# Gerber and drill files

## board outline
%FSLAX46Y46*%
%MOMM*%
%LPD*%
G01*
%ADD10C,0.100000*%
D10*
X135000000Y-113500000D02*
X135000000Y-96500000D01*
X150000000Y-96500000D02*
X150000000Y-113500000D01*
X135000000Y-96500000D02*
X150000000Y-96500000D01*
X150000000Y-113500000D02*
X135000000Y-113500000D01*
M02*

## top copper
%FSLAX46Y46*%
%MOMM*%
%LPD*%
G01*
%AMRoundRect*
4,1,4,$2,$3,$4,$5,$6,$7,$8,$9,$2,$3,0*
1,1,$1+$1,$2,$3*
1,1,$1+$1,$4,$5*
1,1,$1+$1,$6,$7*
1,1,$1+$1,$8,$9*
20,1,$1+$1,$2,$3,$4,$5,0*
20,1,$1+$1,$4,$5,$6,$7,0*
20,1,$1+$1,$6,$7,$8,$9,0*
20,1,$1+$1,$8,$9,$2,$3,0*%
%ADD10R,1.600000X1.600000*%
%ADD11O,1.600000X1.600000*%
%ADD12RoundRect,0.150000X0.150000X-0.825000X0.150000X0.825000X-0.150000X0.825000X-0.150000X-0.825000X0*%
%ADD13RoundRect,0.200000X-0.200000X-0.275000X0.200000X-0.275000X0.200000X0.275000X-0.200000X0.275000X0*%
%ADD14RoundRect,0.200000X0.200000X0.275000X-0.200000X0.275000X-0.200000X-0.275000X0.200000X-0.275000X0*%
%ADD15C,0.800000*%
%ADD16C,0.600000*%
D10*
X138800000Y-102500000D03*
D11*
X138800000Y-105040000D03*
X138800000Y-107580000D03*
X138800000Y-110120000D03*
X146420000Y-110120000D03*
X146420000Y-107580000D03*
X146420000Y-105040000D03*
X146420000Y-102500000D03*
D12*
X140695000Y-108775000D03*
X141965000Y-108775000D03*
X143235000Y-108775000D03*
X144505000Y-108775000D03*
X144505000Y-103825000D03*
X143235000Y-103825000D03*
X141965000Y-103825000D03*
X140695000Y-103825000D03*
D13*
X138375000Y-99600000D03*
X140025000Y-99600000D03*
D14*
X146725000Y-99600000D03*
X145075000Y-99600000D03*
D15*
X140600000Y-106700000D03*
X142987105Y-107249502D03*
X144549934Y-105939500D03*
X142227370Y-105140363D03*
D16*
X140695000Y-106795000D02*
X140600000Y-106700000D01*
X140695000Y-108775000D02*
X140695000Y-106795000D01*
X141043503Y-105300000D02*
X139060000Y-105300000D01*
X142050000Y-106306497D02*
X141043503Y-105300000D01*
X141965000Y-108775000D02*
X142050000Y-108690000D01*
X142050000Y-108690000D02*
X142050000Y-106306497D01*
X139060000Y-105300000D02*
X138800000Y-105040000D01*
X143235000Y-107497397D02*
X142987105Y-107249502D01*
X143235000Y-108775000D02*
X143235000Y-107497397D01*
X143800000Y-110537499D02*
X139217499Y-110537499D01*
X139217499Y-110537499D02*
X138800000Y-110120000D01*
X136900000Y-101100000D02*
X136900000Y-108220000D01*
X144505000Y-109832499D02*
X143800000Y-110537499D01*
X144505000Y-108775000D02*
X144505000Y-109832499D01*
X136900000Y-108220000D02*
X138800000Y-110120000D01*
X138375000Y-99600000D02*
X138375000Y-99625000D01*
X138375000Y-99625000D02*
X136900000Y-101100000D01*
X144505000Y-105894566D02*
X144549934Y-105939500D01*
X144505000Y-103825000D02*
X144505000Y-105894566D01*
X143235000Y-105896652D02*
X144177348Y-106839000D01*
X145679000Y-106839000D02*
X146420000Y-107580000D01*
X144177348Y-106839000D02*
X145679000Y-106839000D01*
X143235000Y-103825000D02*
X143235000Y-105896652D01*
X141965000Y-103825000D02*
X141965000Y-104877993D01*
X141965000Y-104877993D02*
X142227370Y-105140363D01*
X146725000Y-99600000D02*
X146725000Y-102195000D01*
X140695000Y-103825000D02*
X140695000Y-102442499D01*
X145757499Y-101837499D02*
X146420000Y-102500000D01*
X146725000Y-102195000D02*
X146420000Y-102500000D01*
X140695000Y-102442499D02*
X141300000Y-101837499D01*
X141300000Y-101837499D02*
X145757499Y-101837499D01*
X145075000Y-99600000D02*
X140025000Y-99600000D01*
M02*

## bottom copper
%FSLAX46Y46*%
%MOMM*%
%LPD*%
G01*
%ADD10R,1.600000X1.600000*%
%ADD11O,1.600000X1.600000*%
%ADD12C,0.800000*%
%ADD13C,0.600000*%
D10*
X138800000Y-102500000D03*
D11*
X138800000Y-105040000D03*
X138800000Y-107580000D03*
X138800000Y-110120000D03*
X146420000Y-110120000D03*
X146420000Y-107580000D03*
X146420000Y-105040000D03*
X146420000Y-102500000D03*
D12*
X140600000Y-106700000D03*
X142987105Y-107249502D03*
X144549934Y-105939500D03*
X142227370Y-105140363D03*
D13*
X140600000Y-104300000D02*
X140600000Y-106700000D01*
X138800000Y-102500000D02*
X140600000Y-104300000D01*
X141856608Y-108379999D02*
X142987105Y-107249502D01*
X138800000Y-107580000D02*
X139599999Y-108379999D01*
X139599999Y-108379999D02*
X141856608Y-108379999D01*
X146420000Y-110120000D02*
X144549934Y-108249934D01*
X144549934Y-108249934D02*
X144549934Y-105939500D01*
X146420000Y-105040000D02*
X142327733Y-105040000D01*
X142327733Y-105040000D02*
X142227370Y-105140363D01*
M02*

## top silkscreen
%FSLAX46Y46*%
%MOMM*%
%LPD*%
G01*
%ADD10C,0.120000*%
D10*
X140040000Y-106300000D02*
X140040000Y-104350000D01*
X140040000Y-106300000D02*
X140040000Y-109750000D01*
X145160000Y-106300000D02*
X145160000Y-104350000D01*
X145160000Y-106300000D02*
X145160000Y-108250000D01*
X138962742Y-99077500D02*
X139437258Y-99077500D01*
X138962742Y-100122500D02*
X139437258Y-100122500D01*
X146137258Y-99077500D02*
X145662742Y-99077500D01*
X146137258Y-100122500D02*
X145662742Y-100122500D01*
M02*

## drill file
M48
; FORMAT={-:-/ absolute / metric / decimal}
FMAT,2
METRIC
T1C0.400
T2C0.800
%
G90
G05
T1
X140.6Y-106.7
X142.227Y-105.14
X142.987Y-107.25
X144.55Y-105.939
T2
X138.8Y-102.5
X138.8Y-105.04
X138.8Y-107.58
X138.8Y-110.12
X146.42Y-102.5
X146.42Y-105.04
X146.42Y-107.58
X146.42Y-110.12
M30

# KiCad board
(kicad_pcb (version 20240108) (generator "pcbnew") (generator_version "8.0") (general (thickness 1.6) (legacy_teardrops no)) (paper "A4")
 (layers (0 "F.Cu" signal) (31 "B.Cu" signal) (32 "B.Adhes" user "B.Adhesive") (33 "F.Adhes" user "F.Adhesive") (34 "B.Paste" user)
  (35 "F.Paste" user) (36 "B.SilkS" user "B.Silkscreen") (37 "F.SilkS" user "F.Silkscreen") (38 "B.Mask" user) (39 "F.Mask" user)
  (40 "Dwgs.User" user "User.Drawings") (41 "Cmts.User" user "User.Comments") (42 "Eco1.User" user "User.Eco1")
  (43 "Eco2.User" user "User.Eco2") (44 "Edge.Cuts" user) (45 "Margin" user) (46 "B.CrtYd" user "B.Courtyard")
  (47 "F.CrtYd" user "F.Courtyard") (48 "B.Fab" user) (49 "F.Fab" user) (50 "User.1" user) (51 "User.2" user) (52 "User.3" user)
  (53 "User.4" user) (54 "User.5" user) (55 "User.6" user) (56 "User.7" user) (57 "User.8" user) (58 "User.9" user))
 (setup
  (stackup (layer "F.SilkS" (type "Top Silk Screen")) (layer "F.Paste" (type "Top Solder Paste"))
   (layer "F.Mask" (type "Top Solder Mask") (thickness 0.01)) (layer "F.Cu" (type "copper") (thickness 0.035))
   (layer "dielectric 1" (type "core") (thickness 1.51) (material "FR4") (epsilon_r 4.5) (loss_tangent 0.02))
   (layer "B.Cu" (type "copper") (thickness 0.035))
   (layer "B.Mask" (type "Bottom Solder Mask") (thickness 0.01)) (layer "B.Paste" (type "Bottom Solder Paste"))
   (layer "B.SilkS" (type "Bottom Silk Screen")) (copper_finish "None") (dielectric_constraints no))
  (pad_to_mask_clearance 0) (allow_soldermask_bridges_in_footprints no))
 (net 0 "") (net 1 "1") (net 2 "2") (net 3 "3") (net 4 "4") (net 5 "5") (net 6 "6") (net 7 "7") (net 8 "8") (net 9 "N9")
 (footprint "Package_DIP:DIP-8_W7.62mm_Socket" (layer "F.Cu") (at 138.8 102.5)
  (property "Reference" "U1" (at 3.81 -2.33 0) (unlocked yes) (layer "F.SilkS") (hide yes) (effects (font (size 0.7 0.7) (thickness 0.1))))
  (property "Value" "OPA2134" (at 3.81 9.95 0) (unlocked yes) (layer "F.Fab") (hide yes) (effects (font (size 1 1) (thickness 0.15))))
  (pad "1" thru_hole rect (at 0 0) (size 1.6 1.6) (drill 0.8) (layers "*.Cu" "*.Mask") (remove_unused_layers no) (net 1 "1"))
  (pad "2" thru_hole oval (at 0 2.54) (size 1.6 1.6) (drill 0.8) (layers "*.Cu" "*.Mask") (remove_unused_layers no) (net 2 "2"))
  (pad "3" thru_hole oval (at 0 5.08) (size 1.6 1.6) (drill 0.8) (layers "*.Cu" "*.Mask") (remove_unused_layers no) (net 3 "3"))
  (pad "4" thru_hole oval (at 0 7.62) (size 1.6 1.6) (drill 0.8) (layers "*.Cu" "*.Mask") (remove_unused_layers no) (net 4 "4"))
  (pad "5" thru_hole oval (at 7.62 7.62) (size 1.6 1.6) (drill 0.8) (layers "*.Cu" "*.Mask") (remove_unused_layers no) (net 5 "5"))
  (pad "6" thru_hole oval (at 7.62 5.08) (size 1.6 1.6) (drill 0.8) (layers "*.Cu" "*.Mask") (remove_unused_layers no) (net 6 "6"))
  (pad "7" thru_hole oval (at 7.62 2.54) (size 1.6 1.6) (drill 0.8) (layers "*.Cu" "*.Mask") (remove_unused_layers no) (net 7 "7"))
  (pad "8" thru_hole oval (at 7.62 0) (size 1.6 1.6) (drill 0.8) (layers "*.Cu" "*.Mask") (remove_unused_layers no) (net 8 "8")))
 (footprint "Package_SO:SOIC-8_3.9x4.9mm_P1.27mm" (layer "F.Cu") (at 142.6 106.3 90)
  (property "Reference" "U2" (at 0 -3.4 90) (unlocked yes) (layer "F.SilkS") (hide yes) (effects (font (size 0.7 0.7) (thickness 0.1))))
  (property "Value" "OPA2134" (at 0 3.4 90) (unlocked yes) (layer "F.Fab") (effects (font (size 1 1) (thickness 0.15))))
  (fp_line (start 0 -2.56) (end 1.95 -2.56) (stroke (width 0.12) (type solid)) (layer "F.SilkS"))
  (fp_line (start 0 -2.56) (end -3.45 -2.56) (stroke (width 0.12) (type solid)) (layer "F.SilkS"))
  (fp_line (start 0 2.56) (end 1.95 2.56) (stroke (width 0.12) (type solid)) (layer "F.SilkS"))
  (fp_line (start 0 2.56) (end -1.95 2.56) (stroke (width 0.12) (type solid)) (layer "F.SilkS"))
  (pad "1" smd roundrect (at -2.475 -1.905 90) (size 1.95 0.6) (layers "F.Cu" "F.Paste" "F.Mask") (roundrect_rratio 0.25) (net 1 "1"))
  (pad "2" smd roundrect (at -2.475 -0.635 90) (size 1.95 0.6) (layers "F.Cu" "F.Paste" "F.Mask") (roundrect_rratio 0.25) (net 2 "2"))
  (pad "3" smd roundrect (at -2.475 0.635 90) (size 1.95 0.6) (layers "F.Cu" "F.Paste" "F.Mask") (roundrect_rratio 0.25) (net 3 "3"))
  (pad "4" smd roundrect (at -2.475 1.905 90) (size 1.95 0.6) (layers "F.Cu" "F.Paste" "F.Mask") (roundrect_rratio 0.25) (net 4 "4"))
  (pad "5" smd roundrect (at 2.475 1.905 90) (size 1.95 0.6) (layers "F.Cu" "F.Paste" "F.Mask") (roundrect_rratio 0.25) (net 5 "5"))
  (pad "6" smd roundrect (at 2.475 0.635 90) (size 1.95 0.6) (layers "F.Cu" "F.Paste" "F.Mask") (roundrect_rratio 0.25) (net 6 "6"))
  (pad "7" smd roundrect (at 2.475 -0.635 90) (size 1.95 0.6) (layers "F.Cu" "F.Paste" "F.Mask") (roundrect_rratio 0.25) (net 7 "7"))
  (pad "8" smd roundrect (at 2.475 -1.905 90) (size 1.95 0.6) (layers "F.Cu" "F.Paste" "F.Mask") (roundrect_rratio 0.25) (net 8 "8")))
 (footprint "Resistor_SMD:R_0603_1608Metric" (layer "F.Cu") (at 139.2 99.6)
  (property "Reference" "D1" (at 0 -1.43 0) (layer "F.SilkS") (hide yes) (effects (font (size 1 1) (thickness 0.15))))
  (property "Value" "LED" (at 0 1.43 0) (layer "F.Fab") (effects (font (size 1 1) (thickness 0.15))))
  (fp_line (start -0.237258 -0.5225) (end 0.237258 -0.5225) (stroke (width 0.12) (type solid)) (layer "F.SilkS"))
  (fp_line (start -0.237258 0.5225) (end 0.237258 0.5225) (stroke (width 0.12) (type solid)) (layer "F.SilkS"))
  (pad "1" smd roundrect (at -0.825 0) (size 0.8 0.95) (layers "F.Cu" "F.Paste" "F.Mask") (roundrect_rratio 0.25) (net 4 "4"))
  (pad "2" smd roundrect (at 0.825 0) (size 0.8 0.95) (layers "F.Cu" "F.Paste" "F.Mask") (roundrect_rratio 0.25) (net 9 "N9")))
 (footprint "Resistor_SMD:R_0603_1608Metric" (layer "F.Cu") (at 145.9 99.6 180)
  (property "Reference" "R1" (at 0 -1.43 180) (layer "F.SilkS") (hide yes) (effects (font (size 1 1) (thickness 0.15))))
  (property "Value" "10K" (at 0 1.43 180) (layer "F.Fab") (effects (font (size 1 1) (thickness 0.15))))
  (fp_line (start -0.237258 0.5225) (end 0.237258 0.5225) (stroke (width 0.12) (type solid)) (layer "F.SilkS"))
  (fp_line (start -0.237258 -0.5225) (end 0.237258 -0.5225) (stroke (width 0.12) (type solid)) (layer "F.SilkS"))
  (pad "1" smd roundrect (at -0.825 0 180) (size 0.8 0.95) (layers "F.Cu" "F.Paste" "F.Mask") (roundrect_rratio 0.25) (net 8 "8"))
  (pad "2" smd roundrect (at 0.825 0 180) (size 0.8 0.95) (layers "F.Cu" "F.Paste" "F.Mask") (roundrect_rratio 0.25) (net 9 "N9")))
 (gr_line (start 135 113.5) (end 135 96.5) (stroke (width 0.1) (type default)) (layer "Edge.Cuts"))
 (gr_line (start 150 96.5) (end 150 113.5) (stroke (width 0.1) (type default)) (layer "Edge.Cuts"))
 (gr_line (start 135 96.5) (end 150 96.5) (stroke (width 0.1) (type default)) (layer "Edge.Cuts"))
 (gr_line (start 150 113.5) (end 135 113.5) (stroke (width 0.1) (type default)) (layer "Edge.Cuts"))
 (segment (start 140.695 106.795) (end 140.6 106.7) (width 0.6) (layer "F.Cu") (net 1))
 (segment (start 140.695 108.775) (end 140.695 106.795) (width 0.6) (layer "F.Cu") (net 1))
 (via (at 140.6 106.7) (size 0.8) (drill 0.4) (layers "F.Cu" "B.Cu") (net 1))
 (segment (start 140.6 104.3) (end 140.6 106.7) (width 0.6) (layer "B.Cu") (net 1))
 (segment (start 138.8 102.5) (end 140.6 104.3) (width 0.6) (layer "B.Cu") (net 1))
 (segment (start 141.043503 105.3) (end 139.06 105.3) (width 0.6) (layer "F.Cu") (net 2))
 (segment (start 142.05 106.306497) (end 141.043503 105.3) (width 0.6) (layer "F.Cu") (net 2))
 (segment (start 141.965 108.775) (end 142.05 108.69) (width 0.6) (layer "F.Cu") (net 2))
 (segment (start 142.05 108.69) (end 142.05 106.306497) (width 0.6) (layer "F.Cu") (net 2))
 (segment (start 139.06 105.3) (end 138.8 105.04) (width 0.6) (layer "F.Cu") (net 2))
 (segment (start 143.235 107.497397) (end 142.987105 107.249502) (width 0.6) (layer "F.Cu") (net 3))
 (segment (start 143.235 108.775) (end 143.235 107.497397) (width 0.6) (layer "F.Cu") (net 3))
 (via (at 142.987105 107.249502) (size 0.8) (drill 0.4) (layers "F.Cu" "B.Cu") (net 3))
 (segment (start 141.856608 108.379999) (end 142.987105 107.249502) (width 0.6) (layer "B.Cu") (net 3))
 (segment (start 138.8 107.58) (end 139.599999 108.379999) (width 0.6) (layer "B.Cu") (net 3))
 (segment (start 139.599999 108.379999) (end 141.856608 108.379999) (width 0.6) (layer "B.Cu") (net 3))
 (segment (start 143.8 110.537499) (end 139.217499 110.537499) (width 0.6) (layer "F.Cu") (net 4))
 (segment (start 139.217499 110.537499) (end 138.8 110.12) (width 0.6) (layer "F.Cu") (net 4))
 (segment (start 136.9 101.1) (end 136.9 108.22) (width 0.6) (layer "F.Cu") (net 4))
 (segment (start 144.505 109.832499) (end 143.8 110.537499) (width 0.6) (layer "F.Cu") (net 4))
 (segment (start 144.505 108.775) (end 144.505 109.832499) (width 0.6) (layer "F.Cu") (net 4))
 (segment (start 136.9 108.22) (end 138.8 110.12) (width 0.6) (layer "F.Cu") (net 4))
 (segment (start 138.375 99.6) (end 138.375 99.625) (width 0.6) (layer "F.Cu") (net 4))
 (segment (start 138.375 99.625) (end 136.9 101.1) (width 0.6) (layer "F.Cu") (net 4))
 (segment (start 144.505 105.894566) (end 144.549934 105.9395) (width 0.6) (layer "F.Cu") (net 5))
 (segment (start 144.505 103.825) (end 144.505 105.894566) (width 0.6) (layer "F.Cu") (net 5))
 (via (at 144.549934 105.9395) (size 0.8) (drill 0.4) (layers "F.Cu" "B.Cu") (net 5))
 (segment (start 146.42 110.12) (end 144.549934 108.249934) (width 0.6) (layer "B.Cu") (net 5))
 (segment (start 144.549934 108.249934) (end 144.549934 105.9395) (width 0.6) (layer "B.Cu") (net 5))
 (segment (start 143.235 105.896652) (end 144.177348 106.839) (width 0.6) (layer "F.Cu") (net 6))
 (segment (start 145.679 106.839) (end 146.42 107.58) (width 0.6) (layer "F.Cu") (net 6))
 (segment (start 144.177348 106.839) (end 145.679 106.839) (width 0.6) (layer "F.Cu") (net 6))
 (segment (start 143.235 103.825) (end 143.235 105.896652) (width 0.6) (layer "F.Cu") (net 6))
 (segment (start 141.965 103.825) (end 141.965 104.877993) (width 0.6) (layer "F.Cu") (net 7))
 (segment (start 141.965 104.877993) (end 142.22737 105.140363) (width 0.6) (layer "F.Cu") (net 7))
 (via (at 142.22737 105.140363) (size 0.8) (drill 0.4) (layers "F.Cu" "B.Cu") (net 7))
 (segment (start 146.42 105.04) (end 142.327733 105.04) (width 0.6) (layer "B.Cu") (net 7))
 (segment (start 142.327733 105.04) (end 142.22737 105.140363) (width 0.6) (layer "B.Cu") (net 7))
 (segment (start 146.725 99.6) (end 146.725 102.195) (width 0.6) (layer "F.Cu") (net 8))
 (segment (start 140.695 103.825) (end 140.695 102.442499) (width 0.6) (layer "F.Cu") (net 8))
 (segment (start 145.757499 101.837499) (end 146.42 102.5) (width 0.6) (layer "F.Cu") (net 8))
 (segment (start 146.725 102.195) (end 146.42 102.5) (width 0.6) (layer "F.Cu") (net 8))
 (segment (start 140.695 102.442499) (end 141.3 101.837499) (width 0.6) (layer "F.Cu") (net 8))
 (segment (start 141.3 101.837499) (end 145.757499 101.837499) (width 0.6) (layer "F.Cu") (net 8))
 (segment (start 145.075 99.6) (end 140.025 99.6) (width 0.6) (layer "F.Cu") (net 9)))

